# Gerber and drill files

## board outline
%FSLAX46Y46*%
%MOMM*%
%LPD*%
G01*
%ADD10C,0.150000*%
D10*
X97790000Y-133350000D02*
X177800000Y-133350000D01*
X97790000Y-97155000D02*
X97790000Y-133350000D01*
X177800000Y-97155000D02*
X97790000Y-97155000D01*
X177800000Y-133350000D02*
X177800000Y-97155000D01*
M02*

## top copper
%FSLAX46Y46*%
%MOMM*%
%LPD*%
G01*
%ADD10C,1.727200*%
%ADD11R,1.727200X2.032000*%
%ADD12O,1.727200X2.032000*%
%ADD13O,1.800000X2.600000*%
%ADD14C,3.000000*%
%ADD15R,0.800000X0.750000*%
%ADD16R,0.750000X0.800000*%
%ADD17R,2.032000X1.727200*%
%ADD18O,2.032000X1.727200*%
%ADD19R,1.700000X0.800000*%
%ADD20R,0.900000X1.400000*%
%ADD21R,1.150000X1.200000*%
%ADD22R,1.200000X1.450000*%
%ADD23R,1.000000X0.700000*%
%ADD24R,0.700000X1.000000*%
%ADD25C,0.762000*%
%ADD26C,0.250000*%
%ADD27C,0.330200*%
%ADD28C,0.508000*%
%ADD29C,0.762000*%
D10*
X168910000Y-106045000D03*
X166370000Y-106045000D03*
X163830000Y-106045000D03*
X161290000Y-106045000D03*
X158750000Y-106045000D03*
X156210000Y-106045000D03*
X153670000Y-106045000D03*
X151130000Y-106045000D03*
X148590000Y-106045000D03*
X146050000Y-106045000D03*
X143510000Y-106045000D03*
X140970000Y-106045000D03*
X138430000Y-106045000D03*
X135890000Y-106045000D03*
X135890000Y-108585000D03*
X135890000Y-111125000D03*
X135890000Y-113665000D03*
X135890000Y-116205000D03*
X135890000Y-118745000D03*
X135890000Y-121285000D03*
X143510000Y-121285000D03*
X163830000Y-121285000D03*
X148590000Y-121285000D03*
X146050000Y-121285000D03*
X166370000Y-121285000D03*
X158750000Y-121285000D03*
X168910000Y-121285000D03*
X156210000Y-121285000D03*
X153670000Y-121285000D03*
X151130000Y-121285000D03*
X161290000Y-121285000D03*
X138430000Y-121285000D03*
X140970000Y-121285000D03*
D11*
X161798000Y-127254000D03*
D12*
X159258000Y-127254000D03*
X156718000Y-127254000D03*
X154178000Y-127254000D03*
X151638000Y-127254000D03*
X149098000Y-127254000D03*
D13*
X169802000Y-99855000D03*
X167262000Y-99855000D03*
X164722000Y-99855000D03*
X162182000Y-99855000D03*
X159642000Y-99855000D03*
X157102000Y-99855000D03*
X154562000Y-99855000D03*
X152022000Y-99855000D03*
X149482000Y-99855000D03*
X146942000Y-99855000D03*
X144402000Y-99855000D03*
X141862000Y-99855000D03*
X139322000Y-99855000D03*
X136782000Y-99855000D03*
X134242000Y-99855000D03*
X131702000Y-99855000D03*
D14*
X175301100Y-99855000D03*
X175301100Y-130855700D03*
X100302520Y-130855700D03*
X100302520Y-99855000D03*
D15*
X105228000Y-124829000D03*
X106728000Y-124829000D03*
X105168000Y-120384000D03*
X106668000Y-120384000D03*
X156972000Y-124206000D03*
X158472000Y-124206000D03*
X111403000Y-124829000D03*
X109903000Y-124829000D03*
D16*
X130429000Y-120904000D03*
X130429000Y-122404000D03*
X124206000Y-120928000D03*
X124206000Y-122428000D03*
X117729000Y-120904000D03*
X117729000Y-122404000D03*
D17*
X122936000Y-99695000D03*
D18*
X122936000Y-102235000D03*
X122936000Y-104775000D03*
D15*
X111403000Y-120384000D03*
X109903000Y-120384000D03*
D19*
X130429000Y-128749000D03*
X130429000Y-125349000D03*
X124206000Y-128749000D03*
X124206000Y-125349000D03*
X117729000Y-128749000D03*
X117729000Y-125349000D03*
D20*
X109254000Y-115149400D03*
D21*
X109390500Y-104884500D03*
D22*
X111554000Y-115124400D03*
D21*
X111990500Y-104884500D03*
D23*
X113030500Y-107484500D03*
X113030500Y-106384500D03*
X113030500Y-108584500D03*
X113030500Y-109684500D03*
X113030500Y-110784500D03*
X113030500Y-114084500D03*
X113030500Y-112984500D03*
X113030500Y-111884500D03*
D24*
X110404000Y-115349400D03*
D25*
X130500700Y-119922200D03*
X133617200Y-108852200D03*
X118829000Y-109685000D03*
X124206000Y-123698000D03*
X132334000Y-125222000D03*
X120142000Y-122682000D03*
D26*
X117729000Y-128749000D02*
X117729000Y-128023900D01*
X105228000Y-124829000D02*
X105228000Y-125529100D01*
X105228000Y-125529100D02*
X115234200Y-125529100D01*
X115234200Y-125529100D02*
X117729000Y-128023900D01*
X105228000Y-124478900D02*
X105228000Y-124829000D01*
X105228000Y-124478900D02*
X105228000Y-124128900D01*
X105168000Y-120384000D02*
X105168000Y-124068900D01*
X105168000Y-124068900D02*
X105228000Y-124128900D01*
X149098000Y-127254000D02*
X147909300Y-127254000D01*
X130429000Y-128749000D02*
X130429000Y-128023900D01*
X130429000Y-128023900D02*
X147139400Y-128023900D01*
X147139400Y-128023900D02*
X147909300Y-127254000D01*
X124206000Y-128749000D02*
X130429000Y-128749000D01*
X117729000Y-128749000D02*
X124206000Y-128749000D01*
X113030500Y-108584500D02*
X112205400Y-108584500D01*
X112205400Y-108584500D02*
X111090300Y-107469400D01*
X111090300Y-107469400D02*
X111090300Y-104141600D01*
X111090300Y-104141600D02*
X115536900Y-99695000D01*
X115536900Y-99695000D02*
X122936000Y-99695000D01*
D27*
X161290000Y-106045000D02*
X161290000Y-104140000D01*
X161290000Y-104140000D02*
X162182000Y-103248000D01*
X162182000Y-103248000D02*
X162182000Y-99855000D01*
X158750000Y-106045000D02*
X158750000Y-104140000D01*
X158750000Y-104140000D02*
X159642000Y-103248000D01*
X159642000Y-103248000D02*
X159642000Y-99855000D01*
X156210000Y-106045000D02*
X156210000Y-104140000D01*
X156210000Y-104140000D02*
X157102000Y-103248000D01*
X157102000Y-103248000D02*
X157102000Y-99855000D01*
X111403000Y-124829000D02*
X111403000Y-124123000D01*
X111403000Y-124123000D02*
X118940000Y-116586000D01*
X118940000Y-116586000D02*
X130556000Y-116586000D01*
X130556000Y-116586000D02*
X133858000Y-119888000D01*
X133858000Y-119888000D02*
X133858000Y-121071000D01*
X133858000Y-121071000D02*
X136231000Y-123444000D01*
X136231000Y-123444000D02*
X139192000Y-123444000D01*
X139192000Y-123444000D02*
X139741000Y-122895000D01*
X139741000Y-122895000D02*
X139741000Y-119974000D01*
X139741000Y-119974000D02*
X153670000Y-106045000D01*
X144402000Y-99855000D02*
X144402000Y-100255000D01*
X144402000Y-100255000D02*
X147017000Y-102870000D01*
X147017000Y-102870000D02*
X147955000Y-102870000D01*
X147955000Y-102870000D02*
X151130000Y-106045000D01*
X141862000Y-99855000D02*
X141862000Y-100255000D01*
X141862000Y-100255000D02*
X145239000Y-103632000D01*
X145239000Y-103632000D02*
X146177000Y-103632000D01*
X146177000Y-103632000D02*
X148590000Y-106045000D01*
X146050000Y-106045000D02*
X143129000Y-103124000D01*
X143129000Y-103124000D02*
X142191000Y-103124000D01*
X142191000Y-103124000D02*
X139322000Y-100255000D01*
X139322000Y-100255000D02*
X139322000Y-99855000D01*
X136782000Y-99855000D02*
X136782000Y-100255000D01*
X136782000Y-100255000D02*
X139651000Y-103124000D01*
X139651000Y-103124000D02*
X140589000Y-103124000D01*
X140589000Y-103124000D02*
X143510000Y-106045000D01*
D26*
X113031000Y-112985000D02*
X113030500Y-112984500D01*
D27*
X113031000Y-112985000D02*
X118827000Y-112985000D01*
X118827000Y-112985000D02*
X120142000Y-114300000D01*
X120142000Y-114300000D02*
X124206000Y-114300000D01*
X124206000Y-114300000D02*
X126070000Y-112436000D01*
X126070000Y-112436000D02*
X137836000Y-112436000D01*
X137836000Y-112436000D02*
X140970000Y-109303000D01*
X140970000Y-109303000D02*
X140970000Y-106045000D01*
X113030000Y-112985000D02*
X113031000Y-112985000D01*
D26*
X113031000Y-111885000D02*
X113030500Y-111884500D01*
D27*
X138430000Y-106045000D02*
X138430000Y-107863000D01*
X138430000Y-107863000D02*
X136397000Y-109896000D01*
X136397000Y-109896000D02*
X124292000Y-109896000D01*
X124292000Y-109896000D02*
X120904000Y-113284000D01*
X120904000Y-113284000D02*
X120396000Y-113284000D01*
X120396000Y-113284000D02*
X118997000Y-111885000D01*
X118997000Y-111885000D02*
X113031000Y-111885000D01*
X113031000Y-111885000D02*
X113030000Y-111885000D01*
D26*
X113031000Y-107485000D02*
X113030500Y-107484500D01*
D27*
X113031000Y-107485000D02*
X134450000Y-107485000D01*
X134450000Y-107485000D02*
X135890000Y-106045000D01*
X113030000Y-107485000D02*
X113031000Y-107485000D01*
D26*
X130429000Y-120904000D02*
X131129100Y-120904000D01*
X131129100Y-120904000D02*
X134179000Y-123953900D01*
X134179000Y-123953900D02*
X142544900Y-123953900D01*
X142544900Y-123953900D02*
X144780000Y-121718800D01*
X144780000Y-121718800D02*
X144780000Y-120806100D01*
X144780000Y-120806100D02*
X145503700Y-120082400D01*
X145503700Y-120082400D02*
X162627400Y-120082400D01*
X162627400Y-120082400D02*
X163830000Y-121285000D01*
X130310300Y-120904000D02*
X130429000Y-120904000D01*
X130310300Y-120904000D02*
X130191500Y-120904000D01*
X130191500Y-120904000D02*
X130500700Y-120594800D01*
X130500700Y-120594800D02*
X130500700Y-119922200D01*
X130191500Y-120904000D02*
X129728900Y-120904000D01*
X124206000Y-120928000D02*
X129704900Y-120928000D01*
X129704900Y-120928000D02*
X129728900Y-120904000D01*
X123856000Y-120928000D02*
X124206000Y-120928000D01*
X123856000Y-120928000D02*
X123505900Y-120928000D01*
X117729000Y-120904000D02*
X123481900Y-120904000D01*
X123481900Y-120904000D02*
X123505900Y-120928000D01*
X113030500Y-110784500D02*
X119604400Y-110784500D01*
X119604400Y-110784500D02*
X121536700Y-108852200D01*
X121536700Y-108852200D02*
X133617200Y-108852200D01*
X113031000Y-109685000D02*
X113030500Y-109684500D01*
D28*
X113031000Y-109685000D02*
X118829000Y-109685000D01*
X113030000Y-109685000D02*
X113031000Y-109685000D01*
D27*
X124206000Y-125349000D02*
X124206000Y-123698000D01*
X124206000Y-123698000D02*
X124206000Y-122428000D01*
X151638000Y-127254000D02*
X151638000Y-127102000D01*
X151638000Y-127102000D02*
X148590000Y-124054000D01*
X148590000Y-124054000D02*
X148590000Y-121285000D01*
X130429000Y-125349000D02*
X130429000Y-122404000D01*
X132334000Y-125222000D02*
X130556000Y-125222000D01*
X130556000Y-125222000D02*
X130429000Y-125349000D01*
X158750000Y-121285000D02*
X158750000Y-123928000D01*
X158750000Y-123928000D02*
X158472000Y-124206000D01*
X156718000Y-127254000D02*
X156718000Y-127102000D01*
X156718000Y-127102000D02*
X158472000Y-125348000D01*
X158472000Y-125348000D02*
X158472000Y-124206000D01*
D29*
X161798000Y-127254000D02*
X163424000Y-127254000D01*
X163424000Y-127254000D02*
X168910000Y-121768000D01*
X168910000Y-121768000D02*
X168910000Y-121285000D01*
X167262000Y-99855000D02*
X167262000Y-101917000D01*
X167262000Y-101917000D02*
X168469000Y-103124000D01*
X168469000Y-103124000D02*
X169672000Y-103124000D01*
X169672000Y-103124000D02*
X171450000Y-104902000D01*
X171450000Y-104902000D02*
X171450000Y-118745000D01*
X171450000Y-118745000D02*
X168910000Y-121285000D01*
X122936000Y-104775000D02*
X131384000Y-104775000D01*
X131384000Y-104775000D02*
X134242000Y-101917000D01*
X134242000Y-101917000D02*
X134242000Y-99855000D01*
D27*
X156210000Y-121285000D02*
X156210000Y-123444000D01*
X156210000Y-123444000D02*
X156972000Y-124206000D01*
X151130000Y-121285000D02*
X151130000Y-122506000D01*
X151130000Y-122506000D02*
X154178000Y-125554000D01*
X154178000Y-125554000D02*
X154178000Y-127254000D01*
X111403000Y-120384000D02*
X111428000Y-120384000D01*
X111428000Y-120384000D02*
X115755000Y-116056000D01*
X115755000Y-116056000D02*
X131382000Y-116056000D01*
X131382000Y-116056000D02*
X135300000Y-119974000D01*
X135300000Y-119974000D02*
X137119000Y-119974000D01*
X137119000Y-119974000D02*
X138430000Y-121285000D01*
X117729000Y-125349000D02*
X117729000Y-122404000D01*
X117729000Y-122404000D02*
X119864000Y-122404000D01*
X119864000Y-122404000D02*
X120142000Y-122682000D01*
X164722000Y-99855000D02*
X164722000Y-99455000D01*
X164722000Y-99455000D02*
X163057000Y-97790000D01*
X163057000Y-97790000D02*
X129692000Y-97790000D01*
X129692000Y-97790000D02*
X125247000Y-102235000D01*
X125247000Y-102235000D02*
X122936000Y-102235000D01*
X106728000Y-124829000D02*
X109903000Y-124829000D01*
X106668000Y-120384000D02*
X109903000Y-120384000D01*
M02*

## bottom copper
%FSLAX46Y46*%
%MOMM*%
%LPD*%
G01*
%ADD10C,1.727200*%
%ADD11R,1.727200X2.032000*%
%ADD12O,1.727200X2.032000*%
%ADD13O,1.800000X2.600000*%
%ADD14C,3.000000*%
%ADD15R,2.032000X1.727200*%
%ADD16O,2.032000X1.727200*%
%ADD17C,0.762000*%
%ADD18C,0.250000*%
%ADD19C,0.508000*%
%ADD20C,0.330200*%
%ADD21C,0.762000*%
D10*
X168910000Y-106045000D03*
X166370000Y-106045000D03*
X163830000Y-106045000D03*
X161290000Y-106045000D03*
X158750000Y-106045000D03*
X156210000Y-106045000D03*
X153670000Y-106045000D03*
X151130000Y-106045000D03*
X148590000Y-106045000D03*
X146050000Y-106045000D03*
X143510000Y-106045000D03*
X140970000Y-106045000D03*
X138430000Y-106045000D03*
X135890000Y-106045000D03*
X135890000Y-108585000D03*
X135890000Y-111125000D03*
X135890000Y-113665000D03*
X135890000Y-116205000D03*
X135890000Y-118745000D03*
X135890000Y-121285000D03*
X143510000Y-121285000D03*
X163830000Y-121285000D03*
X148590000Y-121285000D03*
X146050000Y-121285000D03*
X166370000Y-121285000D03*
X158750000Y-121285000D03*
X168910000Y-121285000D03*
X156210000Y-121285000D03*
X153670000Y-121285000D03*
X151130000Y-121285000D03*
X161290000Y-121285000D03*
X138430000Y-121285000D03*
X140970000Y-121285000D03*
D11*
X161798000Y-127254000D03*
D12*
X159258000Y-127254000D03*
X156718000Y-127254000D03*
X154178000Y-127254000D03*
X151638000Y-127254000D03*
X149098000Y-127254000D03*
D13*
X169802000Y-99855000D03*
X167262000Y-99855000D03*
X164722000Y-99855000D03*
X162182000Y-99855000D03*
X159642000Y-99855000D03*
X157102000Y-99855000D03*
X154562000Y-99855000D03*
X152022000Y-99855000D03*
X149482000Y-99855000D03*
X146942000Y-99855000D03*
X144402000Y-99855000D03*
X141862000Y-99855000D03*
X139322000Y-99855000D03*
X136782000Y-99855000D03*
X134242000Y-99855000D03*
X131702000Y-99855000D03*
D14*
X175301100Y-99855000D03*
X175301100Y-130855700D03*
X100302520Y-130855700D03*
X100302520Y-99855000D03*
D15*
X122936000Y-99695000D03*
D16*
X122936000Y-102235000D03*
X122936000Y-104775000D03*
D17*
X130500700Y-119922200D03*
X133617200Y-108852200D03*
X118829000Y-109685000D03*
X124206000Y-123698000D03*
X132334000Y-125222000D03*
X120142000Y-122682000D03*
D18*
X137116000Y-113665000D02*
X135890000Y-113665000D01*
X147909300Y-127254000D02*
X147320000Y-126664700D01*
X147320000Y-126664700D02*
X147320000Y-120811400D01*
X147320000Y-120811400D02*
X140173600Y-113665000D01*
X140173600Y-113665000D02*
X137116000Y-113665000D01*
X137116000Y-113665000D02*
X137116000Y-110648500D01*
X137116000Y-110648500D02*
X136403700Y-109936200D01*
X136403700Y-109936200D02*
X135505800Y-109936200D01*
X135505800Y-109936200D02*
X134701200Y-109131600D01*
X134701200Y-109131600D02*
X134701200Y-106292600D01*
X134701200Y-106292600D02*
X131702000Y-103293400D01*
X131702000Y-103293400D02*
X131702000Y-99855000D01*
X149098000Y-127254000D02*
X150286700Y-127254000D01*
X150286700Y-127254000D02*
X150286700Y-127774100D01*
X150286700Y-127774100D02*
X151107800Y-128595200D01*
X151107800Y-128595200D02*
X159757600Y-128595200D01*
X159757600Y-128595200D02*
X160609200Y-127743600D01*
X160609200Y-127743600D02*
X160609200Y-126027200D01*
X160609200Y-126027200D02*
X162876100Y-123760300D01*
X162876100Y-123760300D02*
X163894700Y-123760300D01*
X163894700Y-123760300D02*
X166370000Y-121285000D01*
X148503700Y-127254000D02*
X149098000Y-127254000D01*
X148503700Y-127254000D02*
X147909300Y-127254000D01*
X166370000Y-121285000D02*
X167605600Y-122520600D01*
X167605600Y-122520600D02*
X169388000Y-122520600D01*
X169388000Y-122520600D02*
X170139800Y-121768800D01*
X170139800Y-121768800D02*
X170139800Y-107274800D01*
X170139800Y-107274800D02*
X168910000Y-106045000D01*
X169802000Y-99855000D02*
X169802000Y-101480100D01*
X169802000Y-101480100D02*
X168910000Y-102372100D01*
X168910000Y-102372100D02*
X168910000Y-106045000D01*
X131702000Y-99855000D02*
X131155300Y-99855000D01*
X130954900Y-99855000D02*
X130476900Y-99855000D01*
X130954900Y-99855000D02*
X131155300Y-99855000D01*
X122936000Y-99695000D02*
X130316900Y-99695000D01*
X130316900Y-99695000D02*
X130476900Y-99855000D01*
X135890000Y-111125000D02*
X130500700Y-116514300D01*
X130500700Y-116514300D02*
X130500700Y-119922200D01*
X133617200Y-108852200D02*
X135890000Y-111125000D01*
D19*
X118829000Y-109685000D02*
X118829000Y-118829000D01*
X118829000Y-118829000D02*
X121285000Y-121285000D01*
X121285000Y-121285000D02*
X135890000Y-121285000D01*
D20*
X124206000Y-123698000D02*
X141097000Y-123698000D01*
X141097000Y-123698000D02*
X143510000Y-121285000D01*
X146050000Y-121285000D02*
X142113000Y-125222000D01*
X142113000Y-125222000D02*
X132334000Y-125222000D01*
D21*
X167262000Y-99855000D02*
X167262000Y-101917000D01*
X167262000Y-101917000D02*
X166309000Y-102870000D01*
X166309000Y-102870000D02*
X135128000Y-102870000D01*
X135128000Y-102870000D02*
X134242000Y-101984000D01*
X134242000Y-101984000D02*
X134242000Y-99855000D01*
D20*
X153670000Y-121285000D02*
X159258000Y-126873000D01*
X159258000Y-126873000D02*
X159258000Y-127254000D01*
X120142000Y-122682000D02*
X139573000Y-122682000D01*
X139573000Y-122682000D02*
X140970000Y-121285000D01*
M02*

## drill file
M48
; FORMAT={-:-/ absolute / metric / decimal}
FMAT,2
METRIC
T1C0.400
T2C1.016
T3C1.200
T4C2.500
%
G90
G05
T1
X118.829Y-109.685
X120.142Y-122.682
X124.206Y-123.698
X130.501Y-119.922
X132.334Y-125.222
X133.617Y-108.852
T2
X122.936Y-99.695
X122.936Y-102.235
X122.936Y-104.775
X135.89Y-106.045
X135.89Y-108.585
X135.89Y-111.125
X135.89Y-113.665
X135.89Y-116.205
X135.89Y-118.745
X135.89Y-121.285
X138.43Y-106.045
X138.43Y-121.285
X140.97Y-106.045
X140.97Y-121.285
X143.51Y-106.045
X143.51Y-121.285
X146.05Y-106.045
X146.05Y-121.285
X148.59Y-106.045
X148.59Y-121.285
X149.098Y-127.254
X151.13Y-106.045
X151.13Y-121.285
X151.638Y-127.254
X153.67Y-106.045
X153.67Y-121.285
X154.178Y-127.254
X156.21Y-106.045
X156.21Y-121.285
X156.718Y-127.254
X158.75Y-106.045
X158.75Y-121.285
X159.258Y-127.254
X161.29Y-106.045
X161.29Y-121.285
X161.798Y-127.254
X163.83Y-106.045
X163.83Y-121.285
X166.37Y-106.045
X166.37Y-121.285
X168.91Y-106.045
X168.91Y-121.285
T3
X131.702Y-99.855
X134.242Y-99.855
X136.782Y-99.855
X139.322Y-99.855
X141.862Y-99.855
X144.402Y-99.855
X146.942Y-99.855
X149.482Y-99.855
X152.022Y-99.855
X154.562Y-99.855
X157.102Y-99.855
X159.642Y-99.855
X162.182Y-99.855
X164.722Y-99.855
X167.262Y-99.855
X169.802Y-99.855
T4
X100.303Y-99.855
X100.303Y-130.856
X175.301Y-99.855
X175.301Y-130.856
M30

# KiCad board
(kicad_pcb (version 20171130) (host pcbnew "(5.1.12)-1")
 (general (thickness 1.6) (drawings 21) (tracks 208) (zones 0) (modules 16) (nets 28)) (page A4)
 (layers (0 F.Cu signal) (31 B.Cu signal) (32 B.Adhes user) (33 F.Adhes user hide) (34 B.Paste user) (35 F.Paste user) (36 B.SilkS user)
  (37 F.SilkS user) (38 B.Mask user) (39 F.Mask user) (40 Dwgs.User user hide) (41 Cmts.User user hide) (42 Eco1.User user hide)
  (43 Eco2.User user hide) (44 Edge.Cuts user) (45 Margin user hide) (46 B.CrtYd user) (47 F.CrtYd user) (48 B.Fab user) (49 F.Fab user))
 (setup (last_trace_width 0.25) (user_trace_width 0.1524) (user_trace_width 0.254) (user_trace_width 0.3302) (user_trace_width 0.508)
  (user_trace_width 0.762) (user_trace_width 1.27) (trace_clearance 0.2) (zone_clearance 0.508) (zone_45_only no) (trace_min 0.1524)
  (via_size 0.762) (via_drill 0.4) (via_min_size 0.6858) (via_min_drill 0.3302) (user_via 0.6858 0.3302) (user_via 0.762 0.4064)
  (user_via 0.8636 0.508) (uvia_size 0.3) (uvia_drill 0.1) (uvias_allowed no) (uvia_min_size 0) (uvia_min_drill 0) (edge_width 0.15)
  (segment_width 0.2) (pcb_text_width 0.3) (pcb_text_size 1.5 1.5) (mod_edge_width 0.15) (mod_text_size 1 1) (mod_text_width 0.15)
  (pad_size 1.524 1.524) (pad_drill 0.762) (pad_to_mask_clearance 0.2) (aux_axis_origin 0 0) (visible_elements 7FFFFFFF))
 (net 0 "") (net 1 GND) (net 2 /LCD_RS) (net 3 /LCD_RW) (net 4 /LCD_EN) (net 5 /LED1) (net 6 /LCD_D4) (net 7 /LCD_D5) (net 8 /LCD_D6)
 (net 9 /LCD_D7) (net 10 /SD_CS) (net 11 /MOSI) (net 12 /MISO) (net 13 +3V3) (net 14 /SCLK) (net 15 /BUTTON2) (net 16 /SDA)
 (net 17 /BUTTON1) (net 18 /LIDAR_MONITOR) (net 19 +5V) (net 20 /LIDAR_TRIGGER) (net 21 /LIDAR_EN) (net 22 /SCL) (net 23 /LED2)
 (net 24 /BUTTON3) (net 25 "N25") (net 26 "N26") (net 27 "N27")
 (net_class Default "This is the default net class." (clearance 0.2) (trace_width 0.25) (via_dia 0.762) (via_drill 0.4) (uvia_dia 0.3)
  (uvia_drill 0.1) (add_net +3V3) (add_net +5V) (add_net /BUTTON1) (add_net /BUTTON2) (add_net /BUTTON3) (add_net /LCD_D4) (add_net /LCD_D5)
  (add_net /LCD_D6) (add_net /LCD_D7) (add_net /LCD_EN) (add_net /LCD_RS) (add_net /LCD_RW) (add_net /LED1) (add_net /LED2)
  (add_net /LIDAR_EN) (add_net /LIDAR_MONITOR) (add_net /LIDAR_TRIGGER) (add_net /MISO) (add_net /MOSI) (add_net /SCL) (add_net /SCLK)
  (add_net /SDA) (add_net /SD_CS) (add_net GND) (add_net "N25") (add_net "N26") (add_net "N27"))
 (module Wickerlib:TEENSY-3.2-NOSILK (layer F.Cu) (at 158.75 116.205 270)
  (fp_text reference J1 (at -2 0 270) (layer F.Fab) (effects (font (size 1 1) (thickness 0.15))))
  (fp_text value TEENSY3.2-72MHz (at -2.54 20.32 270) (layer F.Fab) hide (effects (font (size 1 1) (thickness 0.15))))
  (pad G1 thru_hole circle (at -10.16 -10.16 270) (size 1.7272 1.7272) (drill 1.016) (layers *.Cu *.Mask F.SilkS) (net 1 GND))
  (pad 0 thru_hole circle (at -10.16 -7.62 270) (size 1.7272 1.7272) (drill 1.016) (layers *.Cu *.Mask F.SilkS))
  (pad 1 thru_hole circle (at -10.16 -5.08 270) (size 1.7272 1.7272) (drill 1.016) (layers *.Cu *.Mask F.SilkS))
  (pad 2 thru_hole circle (at -10.16 -2.54 270) (size 1.7272 1.7272) (drill 1.016) (layers *.Cu *.Mask F.SilkS) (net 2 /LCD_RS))
  (pad 3 thru_hole circle (at -10.16 0 270) (size 1.7272 1.7272) (drill 1.016) (layers *.Cu *.Mask F.SilkS) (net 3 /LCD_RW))
  (pad 4 thru_hole circle (at -10.16 2.54 270) (size 1.7272 1.7272) (drill 1.016) (layers *.Cu *.Mask F.SilkS) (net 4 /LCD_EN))
  (pad 5 thru_hole circle (at -10.16 5.08 270) (size 1.7272 1.7272) (drill 1.016) (layers *.Cu *.Mask F.SilkS) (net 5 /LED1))
  (pad 6 thru_hole circle (at -10.16 7.62 270) (size 1.7272 1.7272) (drill 1.016) (layers *.Cu *.Mask F.SilkS) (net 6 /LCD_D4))
  (pad 7 thru_hole circle (at -10.16 10.16 270) (size 1.7272 1.7272) (drill 1.016) (layers *.Cu *.Mask F.SilkS) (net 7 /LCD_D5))
  (pad 8 thru_hole circle (at -10.16 12.7 270) (size 1.7272 1.7272) (drill 1.016) (layers *.Cu *.Mask F.SilkS) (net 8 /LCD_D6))
  (pad 9 thru_hole circle (at -10.16 15.24 270) (size 1.7272 1.7272) (drill 1.016) (layers *.Cu *.Mask F.SilkS) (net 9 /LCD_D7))
  (pad 10 thru_hole circle (at -10.16 17.78 270) (size 1.7272 1.7272) (drill 1.016) (layers *.Cu *.Mask F.SilkS) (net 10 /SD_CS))
  (pad 11 thru_hole circle (at -10.16 20.32 270) (size 1.7272 1.7272) (drill 1.016) (layers *.Cu *.Mask F.SilkS) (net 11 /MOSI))
  (pad 12 thru_hole circle (at -10.16 22.86 270) (size 1.7272 1.7272) (drill 1.016) (layers *.Cu *.Mask F.SilkS) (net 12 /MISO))
  (pad VBAT thru_hole circle (at -7.62 22.86 270) (size 1.7272 1.7272) (drill 1.016) (layers *.Cu *.Mask F.SilkS))
  (pad 3V1 thru_hole circle (at -5.08 22.86 270) (size 1.7272 1.7272) (drill 1.016) (layers *.Cu *.Mask F.SilkS) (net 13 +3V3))
  (pad G2 thru_hole circle (at -2.54 22.86 270) (size 1.7272 1.7272) (drill 1.016) (layers *.Cu *.Mask F.SilkS) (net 1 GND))
  (pad PGM thru_hole circle (at 0 22.86 270) (size 1.7272 1.7272) (drill 1.016) (layers *.Cu *.Mask F.SilkS))
  (pad DAC thru_hole circle (at 2.54 22.86 270) (size 1.7272 1.7272) (drill 1.016) (layers *.Cu *.Mask F.SilkS))
  (pad 13 thru_hole circle (at 5.08 22.86 270) (size 1.7272 1.7272) (drill 1.016) (layers *.Cu *.Mask F.SilkS) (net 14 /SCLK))
  (pad 16 thru_hole circle (at 5.08 15.24 270) (size 1.7272 1.7272) (drill 1.016) (layers *.Cu *.Mask F.SilkS) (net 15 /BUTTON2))
  (pad 3V2 thru_hole circle (at 5.08 -5.08 270) (size 1.7272 1.7272) (drill 1.016) (layers *.Cu *.Mask F.SilkS) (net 13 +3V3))
  (pad 18 thru_hole circle (at 5.08 10.16 270) (size 1.7272 1.7272) (drill 1.016) (layers *.Cu *.Mask F.SilkS) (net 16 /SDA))
  (pad 17 thru_hole circle (at 5.08 12.7 270) (size 1.7272 1.7272) (drill 1.016) (layers *.Cu *.Mask F.SilkS) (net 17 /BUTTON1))
  (pad AG thru_hole circle (at 5.08 -7.62 270) (size 1.7272 1.7272) (drill 1.016) (layers *.Cu *.Mask F.SilkS) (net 1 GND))
  (pad 22 thru_hole circle (at 5.08 0 270) (size 1.7272 1.7272) (drill 1.016) (layers *.Cu *.Mask F.SilkS) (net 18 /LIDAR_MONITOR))
  (pad VIN thru_hole circle (at 5.08 -10.16 270) (size 1.7272 1.7272) (drill 1.016) (layers *.Cu *.Mask F.SilkS) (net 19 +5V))
  (pad 21 thru_hole circle (at 5.08 2.54 270) (size 1.7272 1.7272) (drill 1.016) (layers *.Cu *.Mask F.SilkS) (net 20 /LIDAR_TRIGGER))
  (pad 20 thru_hole circle (at 5.08 5.08 270) (size 1.7272 1.7272) (drill 1.016) (layers *.Cu *.Mask F.SilkS) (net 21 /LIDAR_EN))
  (pad 19 thru_hole circle (at 5.08 7.62 270) (size 1.7272 1.7272) (drill 1.016) (layers *.Cu *.Mask F.SilkS) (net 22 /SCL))
  (pad 23 thru_hole circle (at 5.08 -2.54 270) (size 1.7272 1.7272) (drill 1.016) (layers *.Cu *.Mask F.SilkS))
  (pad 14 thru_hole circle (at 5.08 20.32 270) (size 1.7272 1.7272) (drill 1.016) (layers *.Cu *.Mask F.SilkS) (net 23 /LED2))
  (pad 15 thru_hole circle (at 5.08 17.78 270) (size 1.7272 1.7272) (drill 1.016) (layers *.Cu *.Mask F.SilkS) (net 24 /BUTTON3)))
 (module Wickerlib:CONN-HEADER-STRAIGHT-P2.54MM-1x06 (layer F.Cu) (at 161.798 127.254 270)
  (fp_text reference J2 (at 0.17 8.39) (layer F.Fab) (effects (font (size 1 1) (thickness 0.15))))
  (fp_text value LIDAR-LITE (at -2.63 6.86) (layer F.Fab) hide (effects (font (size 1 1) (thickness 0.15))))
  (pad 1 thru_hole rect (at 0 0 270) (size 2.032 1.7272) (drill 1.016) (layers *.Cu *.Mask F.SilkS) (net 19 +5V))
  (pad 2 thru_hole oval (at 0 2.54 270) (size 2.032 1.7272) (drill 1.016) (layers *.Cu *.Mask F.SilkS) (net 21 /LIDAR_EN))
  (pad 3 thru_hole oval (at 0 5.08 270) (size 2.032 1.7272) (drill 1.016) (layers *.Cu *.Mask F.SilkS) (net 18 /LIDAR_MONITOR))
  (pad 4 thru_hole oval (at 0 7.62 270) (size 2.032 1.7272) (drill 1.016) (layers *.Cu *.Mask F.SilkS) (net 22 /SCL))
  (pad 5 thru_hole oval (at 0 10.16 270) (size 2.032 1.7272) (drill 1.016) (layers *.Cu *.Mask F.SilkS) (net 16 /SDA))
  (pad 6 thru_hole oval (at 0 12.7 270) (size 2.032 1.7272) (drill 1.016) (layers *.Cu *.Mask F.SilkS) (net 1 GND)))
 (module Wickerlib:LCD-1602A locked (layer B.Cu) (at 169.802 99.855 180)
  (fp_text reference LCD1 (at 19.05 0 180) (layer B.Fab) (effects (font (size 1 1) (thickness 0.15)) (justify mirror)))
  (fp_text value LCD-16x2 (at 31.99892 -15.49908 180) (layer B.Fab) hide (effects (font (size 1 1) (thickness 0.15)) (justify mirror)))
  (pad 1 thru_hole oval (at 0 0 180) (size 1.8 2.6) (drill 1.2) (layers *.Cu *.Mask B.SilkS) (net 1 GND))
  (pad 2 thru_hole oval (at 2.54 0 180) (size 1.8 2.6) (drill 1.2) (layers *.Cu *.Mask B.SilkS) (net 19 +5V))
  (pad 3 thru_hole oval (at 5.08 0 180) (size 1.8 2.6) (drill 1.2) (layers *.Cu *.Mask B.SilkS) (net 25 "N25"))
  (pad 4 thru_hole oval (at 7.62 0 180) (size 1.8 2.6) (drill 1.2) (layers *.Cu *.Mask B.SilkS) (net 2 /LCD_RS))
  (pad 5 thru_hole oval (at 10.16 0 180) (size 1.8 2.6) (drill 1.2) (layers *.Cu *.Mask B.SilkS) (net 3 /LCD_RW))
  (pad 6 thru_hole oval (at 12.7 0 180) (size 1.8 2.6) (drill 1.2) (layers *.Cu *.Mask B.SilkS) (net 4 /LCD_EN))
  (pad 7 thru_hole oval (at 15.24 0 180) (size 1.8 2.6) (drill 1.2) (layers *.Cu *.Mask B.SilkS))
  (pad 8 thru_hole oval (at 17.78 0 180) (size 1.8 2.6) (drill 1.2) (layers *.Cu *.Mask B.SilkS))
  (pad 9 thru_hole oval (at 20.32 0 180) (size 1.8 2.6) (drill 1.2) (layers *.Cu *.Mask B.SilkS))
  (pad 10 thru_hole oval (at 22.86 0 180) (size 1.8 2.6) (drill 1.2) (layers *.Cu *.Mask B.SilkS))
  (pad 11 thru_hole oval (at 25.4 0 180) (size 1.8 2.6) (drill 1.2) (layers *.Cu *.Mask B.SilkS) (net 6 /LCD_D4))
  (pad 12 thru_hole oval (at 27.94 0 180) (size 1.8 2.6) (drill 1.2) (layers *.Cu *.Mask B.SilkS) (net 7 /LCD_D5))
  (pad 13 thru_hole oval (at 30.48 0 180) (size 1.8 2.6) (drill 1.2) (layers *.Cu *.Mask B.SilkS) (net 8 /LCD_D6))
  (pad 14 thru_hole oval (at 33.02 0 180) (size 1.8 2.6) (drill 1.2) (layers *.Cu *.Mask B.SilkS) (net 9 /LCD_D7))
  (pad 15 thru_hole oval (at 35.56 0 180) (size 1.8 2.6) (drill 1.2) (layers *.Cu *.Mask B.SilkS) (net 19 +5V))
  (pad 16 thru_hole oval (at 38.1 0 180) (size 1.8 2.6) (drill 1.2) (layers *.Cu *.Mask B.SilkS) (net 1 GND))
  (pad 0 thru_hole circle (at -5.4991 0 180) (size 3 3) (drill 2.5) (layers *.Cu *.Mask B.SilkS))
  (pad 0 thru_hole circle (at -5.4991 -31.0007 180) (size 3 3) (drill 2.5) (layers *.Cu *.Mask B.SilkS))
  (pad 0 thru_hole circle (at 69.49948 -31.0007 180) (size 3 3) (drill 2.5) (layers *.Cu *.Mask B.SilkS))
  (pad 0 thru_hole circle (at 69.49948 0 180) (size 3 3) (drill 2.5) (layers *.Cu *.Mask B.SilkS)))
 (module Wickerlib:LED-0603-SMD (layer F.Cu) (at 105.978 124.829)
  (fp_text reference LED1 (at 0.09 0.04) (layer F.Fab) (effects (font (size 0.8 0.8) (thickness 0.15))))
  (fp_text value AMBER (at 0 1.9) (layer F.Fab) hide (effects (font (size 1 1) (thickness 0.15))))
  (pad 1 smd rect (at -0.75 0) (size 0.8 0.75) (layers F.Cu F.Paste F.Mask) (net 1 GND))
  (pad 2 smd rect (at 0.75 0) (size 0.8 0.75) (layers F.Cu F.Paste F.Mask) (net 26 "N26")))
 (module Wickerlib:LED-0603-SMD (layer F.Cu) (at 105.918 120.384)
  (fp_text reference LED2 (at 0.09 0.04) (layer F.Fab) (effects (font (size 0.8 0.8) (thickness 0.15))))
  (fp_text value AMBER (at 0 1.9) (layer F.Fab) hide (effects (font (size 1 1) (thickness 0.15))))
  (pad 1 smd rect (at -0.75 0) (size 0.8 0.75) (layers F.Cu F.Paste F.Mask) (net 1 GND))
  (pad 2 smd rect (at 0.75 0) (size 0.8 0.75) (layers F.Cu F.Paste F.Mask) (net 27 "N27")))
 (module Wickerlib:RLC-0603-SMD (layer F.Cu) (at 157.722 124.206)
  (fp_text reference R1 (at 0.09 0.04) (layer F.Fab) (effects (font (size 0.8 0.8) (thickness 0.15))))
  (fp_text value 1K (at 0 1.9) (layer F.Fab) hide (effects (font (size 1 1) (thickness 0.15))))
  (pad 1 smd rect (at -0.75 0) (size 0.8 0.75) (layers F.Cu F.Paste F.Mask) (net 20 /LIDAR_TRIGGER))
  (pad 2 smd rect (at 0.75 0) (size 0.8 0.75) (layers F.Cu F.Paste F.Mask) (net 18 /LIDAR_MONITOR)))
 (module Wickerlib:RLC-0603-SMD (layer F.Cu) (at 110.653 124.829 180)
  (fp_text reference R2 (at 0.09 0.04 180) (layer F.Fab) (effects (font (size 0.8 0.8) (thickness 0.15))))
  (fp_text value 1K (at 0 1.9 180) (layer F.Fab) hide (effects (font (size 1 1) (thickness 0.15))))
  (pad 1 smd rect (at -0.75 0 180) (size 0.8 0.75) (layers F.Cu F.Paste F.Mask) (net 5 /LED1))
  (pad 2 smd rect (at 0.75 0 180) (size 0.8 0.75) (layers F.Cu F.Paste F.Mask) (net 26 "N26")))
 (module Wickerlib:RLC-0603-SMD (layer F.Cu) (at 130.429 121.654 270)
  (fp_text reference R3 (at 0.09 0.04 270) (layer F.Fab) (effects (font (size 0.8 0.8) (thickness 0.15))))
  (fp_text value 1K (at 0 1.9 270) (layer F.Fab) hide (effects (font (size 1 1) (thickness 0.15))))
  (pad 1 smd rect (at -0.75 0 270) (size 0.8 0.75) (layers F.Cu F.Paste F.Mask) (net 13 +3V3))
  (pad 2 smd rect (at 0.75 0 270) (size 0.8 0.75) (layers F.Cu F.Paste F.Mask) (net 17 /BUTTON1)))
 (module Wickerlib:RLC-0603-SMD (layer F.Cu) (at 124.206 121.678 270)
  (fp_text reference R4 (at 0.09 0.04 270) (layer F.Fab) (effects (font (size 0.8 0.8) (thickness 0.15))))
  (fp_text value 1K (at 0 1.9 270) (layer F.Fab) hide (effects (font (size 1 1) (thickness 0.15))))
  (pad 1 smd rect (at -0.75 0 270) (size 0.8 0.75) (layers F.Cu F.Paste F.Mask) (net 13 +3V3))
  (pad 2 smd rect (at 0.75 0 270) (size 0.8 0.75) (layers F.Cu F.Paste F.Mask) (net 15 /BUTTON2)))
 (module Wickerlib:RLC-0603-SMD (layer F.Cu) (at 117.729 121.654 270)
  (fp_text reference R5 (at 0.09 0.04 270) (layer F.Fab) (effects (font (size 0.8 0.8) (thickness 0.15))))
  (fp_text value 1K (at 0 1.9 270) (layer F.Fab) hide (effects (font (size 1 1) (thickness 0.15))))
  (pad 1 smd rect (at -0.75 0 270) (size 0.8 0.75) (layers F.Cu F.Paste F.Mask) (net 13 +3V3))
  (pad 2 smd rect (at 0.75 0 270) (size 0.8 0.75) (layers F.Cu F.Paste F.Mask) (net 24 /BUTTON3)))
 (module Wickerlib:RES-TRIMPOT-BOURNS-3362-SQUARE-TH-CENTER (layer F.Cu) (at 122.936 102.235)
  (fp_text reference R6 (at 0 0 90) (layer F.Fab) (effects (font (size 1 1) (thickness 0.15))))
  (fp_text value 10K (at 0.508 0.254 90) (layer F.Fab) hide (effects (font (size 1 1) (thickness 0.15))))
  (pad 1 thru_hole rect (at 0 -2.54) (size 2.032 1.7272) (drill 1.016) (layers *.Cu *.Mask F.SilkS) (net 1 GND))
  (pad 2 thru_hole oval (at 0 0) (size 2.032 1.7272) (drill 1.016) (layers *.Cu *.Mask F.SilkS) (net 25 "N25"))
  (pad 3 thru_hole oval (at 0 2.54) (size 2.032 1.7272) (drill 1.016) (layers *.Cu *.Mask F.SilkS) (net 19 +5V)))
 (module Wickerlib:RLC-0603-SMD (layer F.Cu) (at 110.653 120.384 180)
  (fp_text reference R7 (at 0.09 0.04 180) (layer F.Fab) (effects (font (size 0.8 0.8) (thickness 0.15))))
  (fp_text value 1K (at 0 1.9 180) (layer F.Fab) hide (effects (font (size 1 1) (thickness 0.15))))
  (pad 1 smd rect (at -0.75 0 180) (size 0.8 0.75) (layers F.Cu F.Paste F.Mask) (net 23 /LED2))
  (pad 2 smd rect (at 0.75 0 180) (size 0.8 0.75) (layers F.Cu F.Paste F.Mask) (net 27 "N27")))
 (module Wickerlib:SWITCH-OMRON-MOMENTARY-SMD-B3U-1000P (layer F.Cu) (at 130.429 125.349 270)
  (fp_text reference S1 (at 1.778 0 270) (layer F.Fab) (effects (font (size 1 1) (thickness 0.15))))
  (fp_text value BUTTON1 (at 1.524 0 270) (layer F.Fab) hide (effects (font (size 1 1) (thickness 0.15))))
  (pad 2 smd rect (at 3.4 0 270) (size 0.8 1.7) (layers F.Cu F.Paste F.Mask) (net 1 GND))
  (pad 1 smd rect (at 0 0 270) (size 0.8 1.7) (layers F.Cu F.Paste F.Mask) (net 17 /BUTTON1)))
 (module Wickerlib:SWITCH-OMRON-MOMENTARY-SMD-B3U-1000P (layer F.Cu) (at 124.206 125.349 270)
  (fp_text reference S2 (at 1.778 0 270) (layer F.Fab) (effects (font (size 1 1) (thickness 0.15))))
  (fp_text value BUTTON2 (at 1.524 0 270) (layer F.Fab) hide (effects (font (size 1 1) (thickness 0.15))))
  (pad 2 smd rect (at 3.4 0 270) (size 0.8 1.7) (layers F.Cu F.Paste F.Mask) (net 1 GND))
  (pad 1 smd rect (at 0 0 270) (size 0.8 1.7) (layers F.Cu F.Paste F.Mask) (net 15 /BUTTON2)))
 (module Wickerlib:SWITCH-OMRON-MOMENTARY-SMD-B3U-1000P (layer F.Cu) (at 117.729 125.349 270)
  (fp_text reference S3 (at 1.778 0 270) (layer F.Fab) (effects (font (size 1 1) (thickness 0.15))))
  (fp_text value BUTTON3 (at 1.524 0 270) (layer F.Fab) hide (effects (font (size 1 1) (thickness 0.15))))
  (pad 2 smd rect (at 3.4 0 270) (size 0.8 1.7) (layers F.Cu F.Paste F.Mask) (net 1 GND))
  (pad 1 smd rect (at 0 0 270) (size 0.8 1.7) (layers F.Cu F.Paste F.Mask) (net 24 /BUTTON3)))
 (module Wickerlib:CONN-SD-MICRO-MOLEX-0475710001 (layer F.Cu) (at 114.354 110.298 270)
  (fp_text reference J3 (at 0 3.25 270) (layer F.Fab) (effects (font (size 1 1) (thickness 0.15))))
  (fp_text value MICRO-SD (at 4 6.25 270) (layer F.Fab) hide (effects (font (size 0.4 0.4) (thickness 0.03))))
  (pad G5 smd rect (at 4.8514 5.1 270) (size 1.4 0.9) (layers F.Cu F.Paste F.Mask))
  (pad G2 smd rect (at -5.4135 4.9635 270) (size 1.2 1.15) (layers F.Cu F.Paste F.Mask))
  (pad G3 smd rect (at 4.8264 2.8 270) (size 1.45 1.2) (layers F.Cu F.Paste F.Mask))
  (pad G1 smd rect (at -5.4135 2.3635 270) (size 1.2 1.15) (layers F.Cu F.Paste F.Mask))
  (pad 7 smd rect (at -2.8135 1.3235 270) (size 0.7 1) (layers F.Cu F.Paste F.Mask) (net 12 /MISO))
  (pad 8 smd rect (at -3.9135 1.3235 270) (size 0.7 1) (layers F.Cu F.Paste F.Mask))
  (pad 6 smd rect (at -1.7135 1.3235 270) (size 0.7 1) (layers F.Cu F.Paste F.Mask) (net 1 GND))
  (pad 5 smd rect (at -0.6135 1.3235 270) (size 0.7 1) (layers F.Cu F.Paste F.Mask) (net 14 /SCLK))
  (pad 4 smd rect (at 0.4865 1.3235 270) (size 0.7 1) (layers F.Cu F.Paste F.Mask) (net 13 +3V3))
  (pad 1 smd rect (at 3.7865 1.3235 270) (size 0.7 1) (layers F.Cu F.Paste F.Mask))
  (pad 2 smd rect (at 2.6865 1.3235 270) (size 0.7 1) (layers F.Cu F.Paste F.Mask) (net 10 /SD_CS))
  (pad 3 smd rect (at 1.5865 1.3235 270) (size 0.7 1) (layers F.Cu F.Paste F.Mask) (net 11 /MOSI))
  (pad G4 smd rect (at 5.0514 3.95 270) (size 1 0.7) (layers F.Cu F.Paste F.Mask)))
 (gr_line (start 97.79 133.35) (end 177.8 133.35) (layer Edge.Cuts) (width 0.15))
 (gr_line (start 97.79 97.155) (end 97.79 133.35) (layer Edge.Cuts) (width 0.15))
 (gr_line (start 177.8 97.155) (end 97.79 97.155) (layer Edge.Cuts) (width 0.15))
 (gr_line (start 177.8 133.35) (end 177.8 97.155) (layer Edge.Cuts) (width 0.15))
 (segment (start 137.116 113.665) (end 135.89 113.665) (width 0.25) (layer B.Cu) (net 1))
 (segment (start 147.9093 127.254) (end 147.32 126.6647) (width 0.25) (layer B.Cu) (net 1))
 (segment (start 147.32 126.6647) (end 147.32 120.8114) (width 0.25) (layer B.Cu) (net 1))
 (segment (start 147.32 120.8114) (end 140.1736 113.665) (width 0.25) (layer B.Cu) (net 1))
 (segment (start 140.1736 113.665) (end 137.116 113.665) (width 0.25) (layer B.Cu) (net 1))
 (segment (start 137.116 113.665) (end 137.116 110.6485) (width 0.25) (layer B.Cu) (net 1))
 (segment (start 137.116 110.6485) (end 136.4037 109.9362) (width 0.25) (layer B.Cu) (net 1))
 (segment (start 136.4037 109.9362) (end 135.5058 109.9362) (width 0.25) (layer B.Cu) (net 1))
 (segment (start 135.5058 109.9362) (end 134.7012 109.1316) (width 0.25) (layer B.Cu) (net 1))
 (segment (start 134.7012 109.1316) (end 134.7012 106.2926) (width 0.25) (layer B.Cu) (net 1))
 (segment (start 134.7012 106.2926) (end 131.702 103.2934) (width 0.25) (layer B.Cu) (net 1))
 (segment (start 131.702 103.2934) (end 131.702 99.855) (width 0.25) (layer B.Cu) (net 1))
 (segment (start 149.098 127.254) (end 150.2867 127.254) (width 0.25) (layer B.Cu) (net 1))
 (segment (start 150.2867 127.254) (end 150.2867 127.7741) (width 0.25) (layer B.Cu) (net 1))
 (segment (start 150.2867 127.7741) (end 151.1078 128.5952) (width 0.25) (layer B.Cu) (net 1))
 (segment (start 151.1078 128.5952) (end 159.7576 128.5952) (width 0.25) (layer B.Cu) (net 1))
 (segment (start 159.7576 128.5952) (end 160.6092 127.7436) (width 0.25) (layer B.Cu) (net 1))
 (segment (start 160.6092 127.7436) (end 160.6092 126.0272) (width 0.25) (layer B.Cu) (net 1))
 (segment (start 160.6092 126.0272) (end 162.8761 123.7603) (width 0.25) (layer B.Cu) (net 1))
 (segment (start 162.8761 123.7603) (end 163.8947 123.7603) (width 0.25) (layer B.Cu) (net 1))
 (segment (start 163.8947 123.7603) (end 166.37 121.285) (width 0.25) (layer B.Cu) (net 1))
 (segment (start 148.5037 127.254) (end 149.098 127.254) (width 0.25) (layer B.Cu) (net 1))
 (segment (start 148.5037 127.254) (end 147.9093 127.254) (width 0.25) (layer B.Cu) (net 1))
 (segment (start 166.37 121.285) (end 167.6056 122.5206) (width 0.25) (layer B.Cu) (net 1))
 (segment (start 167.6056 122.5206) (end 169.388 122.5206) (width 0.25) (layer B.Cu) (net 1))
 (segment (start 169.388 122.5206) (end 170.1398 121.7688) (width 0.25) (layer B.Cu) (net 1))
 (segment (start 170.1398 121.7688) (end 170.1398 107.2748) (width 0.25) (layer B.Cu) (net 1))
 (segment (start 170.1398 107.2748) (end 168.91 106.045) (width 0.25) (layer B.Cu) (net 1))
 (segment (start 169.802 99.855) (end 169.802 101.4801) (width 0.25) (layer B.Cu) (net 1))
 (segment (start 169.802 101.4801) (end 168.91 102.3721) (width 0.25) (layer B.Cu) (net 1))
 (segment (start 168.91 102.3721) (end 168.91 106.045) (width 0.25) (layer B.Cu) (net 1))
 (segment (start 131.702 99.855) (end 131.1553 99.855) (width 0.25) (layer B.Cu) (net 1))
 (segment (start 130.9549 99.855) (end 130.4769 99.855) (width 0.25) (layer B.Cu) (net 1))
 (segment (start 130.9549 99.855) (end 131.1553 99.855) (width 0.25) (layer B.Cu) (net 1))
 (segment (start 117.729 128.749) (end 117.729 128.0239) (width 0.25) (layer F.Cu) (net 1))
 (segment (start 105.228 124.829) (end 105.228 125.5291) (width 0.25) (layer F.Cu) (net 1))
 (segment (start 105.228 125.5291) (end 115.2342 125.5291) (width 0.25) (layer F.Cu) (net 1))
 (segment (start 115.2342 125.5291) (end 117.729 128.0239) (width 0.25) (layer F.Cu) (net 1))
 (segment (start 105.228 124.4789) (end 105.228 124.829) (width 0.25) (layer F.Cu) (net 1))
 (segment (start 105.228 124.4789) (end 105.228 124.1289) (width 0.25) (layer F.Cu) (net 1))
 (segment (start 105.168 120.384) (end 105.168 124.0689) (width 0.25) (layer F.Cu) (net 1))
 (segment (start 105.168 124.0689) (end 105.228 124.1289) (width 0.25) (layer F.Cu) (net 1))
 (segment (start 122.936 99.695) (end 130.3169 99.695) (width 0.25) (layer B.Cu) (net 1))
 (segment (start 130.3169 99.695) (end 130.4769 99.855) (width 0.25) (layer B.Cu) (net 1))
 (segment (start 149.098 127.254) (end 147.9093 127.254) (width 0.25) (layer F.Cu) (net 1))
 (segment (start 130.429 128.749) (end 130.429 128.0239) (width 0.25) (layer F.Cu) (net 1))
 (segment (start 130.429 128.0239) (end 147.1394 128.0239) (width 0.25) (layer F.Cu) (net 1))
 (segment (start 147.1394 128.0239) (end 147.9093 127.254) (width 0.25) (layer F.Cu) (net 1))
 (segment (start 124.206 128.749) (end 130.429 128.749) (width 0.25) (layer F.Cu) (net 1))
 (segment (start 117.729 128.749) (end 124.206 128.749) (width 0.25) (layer F.Cu) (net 1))
 (segment (start 113.0305 108.5845) (end 112.2054 108.5845) (width 0.25) (layer F.Cu) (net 1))
 (segment (start 112.2054 108.5845) (end 111.0903 107.4694) (width 0.25) (layer F.Cu) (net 1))
 (segment (start 111.0903 107.4694) (end 111.0903 104.1416) (width 0.25) (layer F.Cu) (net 1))
 (segment (start 111.0903 104.1416) (end 115.5369 99.695) (width 0.25) (layer F.Cu) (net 1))
 (segment (start 115.5369 99.695) (end 122.936 99.695) (width 0.25) (layer F.Cu) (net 1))
 (segment (start 161.29 106.045) (end 161.29 104.14) (width 0.3302) (layer F.Cu) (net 2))
 (segment (start 161.29 104.14) (end 162.182 103.248) (width 0.3302) (layer F.Cu) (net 2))
 (segment (start 162.182 103.248) (end 162.182 99.855) (width 0.3302) (layer F.Cu) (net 2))
 (segment (start 158.75 106.045) (end 158.75 104.14) (width 0.3302) (layer F.Cu) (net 3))
 (segment (start 158.75 104.14) (end 159.642 103.248) (width 0.3302) (layer F.Cu) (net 3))
 (segment (start 159.642 103.248) (end 159.642 99.855) (width 0.3302) (layer F.Cu) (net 3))
 (segment (start 156.21 106.045) (end 156.21 104.14) (width 0.3302) (layer F.Cu) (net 4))
 (segment (start 156.21 104.14) (end 157.102 103.248) (width 0.3302) (layer F.Cu) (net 4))
 (segment (start 157.102 103.248) (end 157.102 99.855) (width 0.3302) (layer F.Cu) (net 4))
 (segment (start 111.403 124.829) (end 111.403 124.123) (width 0.3302) (layer F.Cu) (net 5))
 (segment (start 111.403 124.123) (end 118.94 116.586) (width 0.3302) (layer F.Cu) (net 5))
 (segment (start 118.94 116.586) (end 130.556 116.586) (width 0.3302) (layer F.Cu) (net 5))
 (segment (start 130.556 116.586) (end 133.858 119.888) (width 0.3302) (layer F.Cu) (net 5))
 (segment (start 133.858 119.888) (end 133.858 121.071) (width 0.3302) (layer F.Cu) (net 5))
 (segment (start 133.858 121.071) (end 136.231 123.444) (width 0.3302) (layer F.Cu) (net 5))
 (segment (start 136.231 123.444) (end 139.192 123.444) (width 0.3302) (layer F.Cu) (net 5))
 (segment (start 139.192 123.444) (end 139.741 122.895) (width 0.3302) (layer F.Cu) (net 5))
 (segment (start 139.741 122.895) (end 139.741 119.974) (width 0.3302) (layer F.Cu) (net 5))
 (segment (start 139.741 119.974) (end 153.67 106.045) (width 0.3302) (layer F.Cu) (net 5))
 (segment (start 144.402 99.855) (end 144.402 100.255) (width 0.3302) (layer F.Cu) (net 6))
 (segment (start 144.402 100.255) (end 147.017 102.87) (width 0.3302) (layer F.Cu) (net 6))
 (segment (start 147.017 102.87) (end 147.955 102.87) (width 0.3302) (layer F.Cu) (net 6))
 (segment (start 147.955 102.87) (end 151.13 106.045) (width 0.3302) (layer F.Cu) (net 6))
 (segment (start 141.862 99.855) (end 141.862 100.255) (width 0.3302) (layer F.Cu) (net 7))
 (segment (start 141.862 100.255) (end 145.239 103.632) (width 0.3302) (layer F.Cu) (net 7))
 (segment (start 145.239 103.632) (end 146.177 103.632) (width 0.3302) (layer F.Cu) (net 7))
 (segment (start 146.177 103.632) (end 148.59 106.045) (width 0.3302) (layer F.Cu) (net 7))
 (segment (start 146.05 106.045) (end 143.129 103.124) (width 0.3302) (layer F.Cu) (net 8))
 (segment (start 143.129 103.124) (end 142.191 103.124) (width 0.3302) (layer F.Cu) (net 8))
 (segment (start 142.191 103.124) (end 139.322 100.255) (width 0.3302) (layer F.Cu) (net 8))
 (segment (start 139.322 100.255) (end 139.322 99.855) (width 0.3302) (layer F.Cu) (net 8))
 (segment (start 136.782 99.855) (end 136.782 100.255) (width 0.3302) (layer F.Cu) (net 9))
 (segment (start 136.782 100.255) (end 139.651 103.124) (width 0.3302) (layer F.Cu) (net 9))
 (segment (start 139.651 103.124) (end 140.589 103.124) (width 0.3302) (layer F.Cu) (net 9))
 (segment (start 140.589 103.124) (end 143.51 106.045) (width 0.3302) (layer F.Cu) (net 9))
 (segment (start 113.031 112.985) (end 113.0305 112.9845) (width 0.25) (layer F.Cu) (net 10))
 (segment (start 113.031 112.985) (end 118.827 112.985) (width 0.3302) (layer F.Cu) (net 10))
 (segment (start 118.827 112.985) (end 120.142 114.3) (width 0.3302) (layer F.Cu) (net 10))
 (segment (start 120.142 114.3) (end 124.206 114.3) (width 0.3302) (layer F.Cu) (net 10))
 (segment (start 124.206 114.3) (end 126.07 112.436) (width 0.3302) (layer F.Cu) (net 10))
 (segment (start 126.07 112.436) (end 137.836 112.436) (width 0.3302) (layer F.Cu) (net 10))
 (segment (start 137.836 112.436) (end 140.97 109.303) (width 0.3302) (layer F.Cu) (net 10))
 (segment (start 140.97 109.303) (end 140.97 106.045) (width 0.3302) (layer F.Cu) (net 10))
 (segment (start 113.03 112.985) (end 113.031 112.985) (width 0.3302) (layer F.Cu) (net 10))
 (segment (start 113.031 111.885) (end 113.0305 111.8845) (width 0.25) (layer F.Cu) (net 11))
 (segment (start 138.43 106.045) (end 138.43 107.863) (width 0.3302) (layer F.Cu) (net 11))
 (segment (start 138.43 107.863) (end 136.397 109.896) (width 0.3302) (layer F.Cu) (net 11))
 (segment (start 136.397 109.896) (end 124.292 109.896) (width 0.3302) (layer F.Cu) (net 11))
 (segment (start 124.292 109.896) (end 120.904 113.284) (width 0.3302) (layer F.Cu) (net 11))
 (segment (start 120.904 113.284) (end 120.396 113.284) (width 0.3302) (layer F.Cu) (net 11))
 (segment (start 120.396 113.284) (end 118.997 111.885) (width 0.3302) (layer F.Cu) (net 11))
 (segment (start 118.997 111.885) (end 113.031 111.885) (width 0.3302) (layer F.Cu) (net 11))
 (segment (start 113.031 111.885) (end 113.03 111.885) (width 0.3302) (layer F.Cu) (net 11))
 (segment (start 113.031 107.485) (end 113.0305 107.4845) (width 0.25) (layer F.Cu) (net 12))
 (segment (start 113.031 107.485) (end 134.45 107.485) (width 0.3302) (layer F.Cu) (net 12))
 (segment (start 134.45 107.485) (end 135.89 106.045) (width 0.3302) (layer F.Cu) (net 12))
 (segment (start 113.03 107.485) (end 113.031 107.485) (width 0.3302) (layer F.Cu) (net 12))
 (segment (start 130.429 120.904) (end 131.1291 120.904) (width 0.25) (layer F.Cu) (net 13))
 (segment (start 131.1291 120.904) (end 134.179 123.9539) (width 0.25) (layer F.Cu) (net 13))
 (segment (start 134.179 123.9539) (end 142.5449 123.9539) (width 0.25) (layer F.Cu) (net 13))
 (segment (start 142.5449 123.9539) (end 144.78 121.7188) (width 0.25) (layer F.Cu) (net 13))
 (segment (start 144.78 121.7188) (end 144.78 120.8061) (width 0.25) (layer F.Cu) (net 13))
 (segment (start 144.78 120.8061) (end 145.5037 120.0824) (width 0.25) (layer F.Cu) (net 13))
 (segment (start 145.5037 120.0824) (end 162.6274 120.0824) (width 0.25) (layer F.Cu) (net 13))
 (segment (start 162.6274 120.0824) (end 163.83 121.285) (width 0.25) (layer F.Cu) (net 13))
 (segment (start 130.3103 120.904) (end 130.429 120.904) (width 0.25) (layer F.Cu) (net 13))
 (segment (start 130.3103 120.904) (end 130.1915 120.904) (width 0.25) (layer F.Cu) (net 13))
 (segment (start 135.89 111.125) (end 130.5007 116.5143) (width 0.25) (layer B.Cu) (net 13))
 (segment (start 130.5007 116.5143) (end 130.5007 119.9222) (width 0.25) (layer B.Cu) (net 13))
 (segment (start 130.1915 120.904) (end 130.5007 120.5948) (width 0.25) (layer F.Cu) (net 13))
 (segment (start 130.5007 120.5948) (end 130.5007 119.9222) (width 0.25) (layer F.Cu) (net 13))
 (segment (start 133.6172 108.8522) (end 135.89 111.125) (width 0.25) (layer B.Cu) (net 13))
 (segment (start 130.1915 120.904) (end 129.7289 120.904) (width 0.25) (layer F.Cu) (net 13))
 (segment (start 124.206 120.928) (end 129.7049 120.928) (width 0.25) (layer F.Cu) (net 13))
 (segment (start 129.7049 120.928) (end 129.7289 120.904) (width 0.25) (layer F.Cu) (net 13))
 (segment (start 123.856 120.928) (end 124.206 120.928) (width 0.25) (layer F.Cu) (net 13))
 (segment (start 123.856 120.928) (end 123.5059 120.928) (width 0.25) (layer F.Cu) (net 13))
 (segment (start 117.729 120.904) (end 123.4819 120.904) (width 0.25) (layer F.Cu) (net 13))
 (segment (start 123.4819 120.904) (end 123.5059 120.928) (width 0.25) (layer F.Cu) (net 13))
 (segment (start 113.0305 110.7845) (end 119.6044 110.7845) (width 0.25) (layer F.Cu) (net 13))
 (segment (start 119.6044 110.7845) (end 121.5367 108.8522) (width 0.25) (layer F.Cu) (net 13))
 (segment (start 121.5367 108.8522) (end 133.6172 108.8522) (width 0.25) (layer F.Cu) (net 13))
 (via (at 130.5007 119.9222) (size 0.762) (layers F.Cu B.Cu) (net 13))
 (via (at 133.6172 108.8522) (size 0.762) (layers F.Cu B.Cu) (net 13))
 (segment (start 113.031 109.685) (end 113.0305 109.6845) (width 0.25) (layer F.Cu) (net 14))
 (segment (start 113.031 109.685) (end 118.829 109.685) (width 0.508) (layer F.Cu) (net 14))
 (segment (start 113.03 109.685) (end 113.031 109.685) (width 0.508) (layer F.Cu) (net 14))
 (segment (start 118.829 109.685) (end 118.829 118.829) (width 0.508) (layer B.Cu) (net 14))
 (segment (start 118.829 118.829) (end 121.285 121.285) (width 0.508) (layer B.Cu) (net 14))
 (segment (start 121.285 121.285) (end 135.89 121.285) (width 0.508) (layer B.Cu) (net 14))
 (via (at 118.829 109.685) (size 0.762) (layers F.Cu B.Cu) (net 14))
 (segment (start 124.206 125.349) (end 124.206 123.698) (width 0.3302) (layer F.Cu) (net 15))
 (segment (start 124.206 123.698) (end 124.206 122.428) (width 0.3302) (layer F.Cu) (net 15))
 (segment (start 124.206 123.698) (end 141.097 123.698) (width 0.3302) (layer B.Cu) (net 15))
 (segment (start 141.097 123.698) (end 143.51 121.285) (width 0.3302) (layer B.Cu) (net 15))
 (via (at 124.206 123.698) (size 0.762) (layers F.Cu B.Cu) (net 15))
 (segment (start 151.638 127.254) (end 151.638 127.102) (width 0.3302) (layer F.Cu) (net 16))
 (segment (start 151.638 127.102) (end 148.59 124.054) (width 0.3302) (layer F.Cu) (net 16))
 (segment (start 148.59 124.054) (end 148.59 121.285) (width 0.3302) (layer F.Cu) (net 16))
 (segment (start 130.429 125.349) (end 130.429 122.404) (width 0.3302) (layer F.Cu) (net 17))
 (segment (start 146.05 121.285) (end 142.113 125.222) (width 0.3302) (layer B.Cu) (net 17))
 (segment (start 142.113 125.222) (end 132.334 125.222) (width 0.3302) (layer B.Cu) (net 17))
 (segment (start 132.334 125.222) (end 130.556 125.222) (width 0.3302) (layer F.Cu) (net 17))
 (segment (start 130.556 125.222) (end 130.429 125.349) (width 0.3302) (layer F.Cu) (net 17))
 (via (at 132.334 125.222) (size 0.762) (layers F.Cu B.Cu) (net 17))
 (segment (start 158.75 121.285) (end 158.75 123.928) (width 0.3302) (layer F.Cu) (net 18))
 (segment (start 158.75 123.928) (end 158.472 124.206) (width 0.3302) (layer F.Cu) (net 18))
 (segment (start 156.718 127.254) (end 156.718 127.102) (width 0.3302) (layer F.Cu) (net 18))
 (segment (start 156.718 127.102) (end 158.472 125.348) (width 0.3302) (layer F.Cu) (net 18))
 (segment (start 158.472 125.348) (end 158.472 124.206) (width 0.3302) (layer F.Cu) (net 18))
 (segment (start 161.798 127.254) (end 163.424 127.254) (width 0.762) (layer F.Cu) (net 19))
 (segment (start 163.424 127.254) (end 168.91 121.768) (width 0.762) (layer F.Cu) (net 19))
 (segment (start 168.91 121.768) (end 168.91 121.285) (width 0.762) (layer F.Cu) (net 19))
 (segment (start 167.262 99.855) (end 167.262 101.917) (width 0.762) (layer F.Cu) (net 19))
 (segment (start 167.262 101.917) (end 168.469 103.124) (width 0.762) (layer F.Cu) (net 19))
 (segment (start 168.469 103.124) (end 169.672 103.124) (width 0.762) (layer F.Cu) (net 19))
 (segment (start 169.672 103.124) (end 171.45 104.902) (width 0.762) (layer F.Cu) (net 19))
 (segment (start 171.45 104.902) (end 171.45 118.745) (width 0.762) (layer F.Cu) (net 19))
 (segment (start 171.45 118.745) (end 168.91 121.285) (width 0.762) (layer F.Cu) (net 19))
 (segment (start 167.262 99.855) (end 167.262 101.917) (width 0.762) (layer B.Cu) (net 19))
 (segment (start 167.262 101.917) (end 166.309 102.87) (width 0.762) (layer B.Cu) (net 19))
 (segment (start 166.309 102.87) (end 135.128 102.87) (width 0.762) (layer B.Cu) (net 19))
 (segment (start 135.128 102.87) (end 134.242 101.984) (width 0.762) (layer B.Cu) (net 19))
 (segment (start 134.242 101.984) (end 134.242 99.855) (width 0.762) (layer B.Cu) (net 19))
 (segment (start 122.936 104.775) (end 131.384 104.775) (width 0.762) (layer F.Cu) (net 19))
 (segment (start 131.384 104.775) (end 134.242 101.917) (width 0.762) (layer F.Cu) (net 19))
 (segment (start 134.242 101.917) (end 134.242 99.855) (width 0.762) (layer F.Cu) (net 19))
 (segment (start 156.21 121.285) (end 156.21 123.444) (width 0.3302) (layer F.Cu) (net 20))
 (segment (start 156.21 123.444) (end 156.972 124.206) (width 0.3302) (layer F.Cu) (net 20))
 (segment (start 153.67 121.285) (end 159.258 126.873) (width 0.3302) (layer B.Cu) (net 21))
 (segment (start 159.258 126.873) (end 159.258 127.254) (width 0.3302) (layer B.Cu) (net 21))
 (segment (start 151.13 121.285) (end 151.13 122.506) (width 0.3302) (layer F.Cu) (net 22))
 (segment (start 151.13 122.506) (end 154.178 125.554) (width 0.3302) (layer F.Cu) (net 22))
 (segment (start 154.178 125.554) (end 154.178 127.254) (width 0.3302) (layer F.Cu) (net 22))
 (segment (start 111.403 120.384) (end 111.428 120.384) (width 0.3302) (layer F.Cu) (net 23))
 (segment (start 111.428 120.384) (end 115.755 116.056) (width 0.3302) (layer F.Cu) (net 23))
 (segment (start 115.755 116.056) (end 131.382 116.056) (width 0.3302) (layer F.Cu) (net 23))
 (segment (start 131.382 116.056) (end 135.3 119.974) (width 0.3302) (layer F.Cu) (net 23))
 (segment (start 135.3 119.974) (end 137.119 119.974) (width 0.3302) (layer F.Cu) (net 23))
 (segment (start 137.119 119.974) (end 138.43 121.285) (width 0.3302) (layer F.Cu) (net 23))
 (segment (start 117.729 125.349) (end 117.729 122.404) (width 0.3302) (layer F.Cu) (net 24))
 (segment (start 117.729 122.404) (end 119.864 122.404) (width 0.3302) (layer F.Cu) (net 24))
 (segment (start 119.864 122.404) (end 120.142 122.682) (width 0.3302) (layer F.Cu) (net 24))
 (segment (start 120.142 122.682) (end 139.573 122.682) (width 0.3302) (layer B.Cu) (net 24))
 (segment (start 139.573 122.682) (end 140.97 121.285) (width 0.3302) (layer B.Cu) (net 24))
 (via (at 120.142 122.682) (size 0.762) (layers F.Cu B.Cu) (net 24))
 (segment (start 164.722 99.855) (end 164.722 99.455) (width 0.3302) (layer F.Cu) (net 25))
 (segment (start 164.722 99.455) (end 163.057 97.79) (width 0.3302) (layer F.Cu) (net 25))
 (segment (start 163.057 97.79) (end 129.692 97.79) (width 0.3302) (layer F.Cu) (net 25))
 (segment (start 129.692 97.79) (end 125.247 102.235) (width 0.3302) (layer F.Cu) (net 25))
 (segment (start 125.247 102.235) (end 122.936 102.235) (width 0.3302) (layer F.Cu) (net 25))
 (segment (start 106.728 124.829) (end 109.903 124.829) (width 0.3302) (layer F.Cu) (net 26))
 (segment (start 106.668 120.384) (end 109.903 120.384) (width 0.3302) (layer F.Cu) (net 27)))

